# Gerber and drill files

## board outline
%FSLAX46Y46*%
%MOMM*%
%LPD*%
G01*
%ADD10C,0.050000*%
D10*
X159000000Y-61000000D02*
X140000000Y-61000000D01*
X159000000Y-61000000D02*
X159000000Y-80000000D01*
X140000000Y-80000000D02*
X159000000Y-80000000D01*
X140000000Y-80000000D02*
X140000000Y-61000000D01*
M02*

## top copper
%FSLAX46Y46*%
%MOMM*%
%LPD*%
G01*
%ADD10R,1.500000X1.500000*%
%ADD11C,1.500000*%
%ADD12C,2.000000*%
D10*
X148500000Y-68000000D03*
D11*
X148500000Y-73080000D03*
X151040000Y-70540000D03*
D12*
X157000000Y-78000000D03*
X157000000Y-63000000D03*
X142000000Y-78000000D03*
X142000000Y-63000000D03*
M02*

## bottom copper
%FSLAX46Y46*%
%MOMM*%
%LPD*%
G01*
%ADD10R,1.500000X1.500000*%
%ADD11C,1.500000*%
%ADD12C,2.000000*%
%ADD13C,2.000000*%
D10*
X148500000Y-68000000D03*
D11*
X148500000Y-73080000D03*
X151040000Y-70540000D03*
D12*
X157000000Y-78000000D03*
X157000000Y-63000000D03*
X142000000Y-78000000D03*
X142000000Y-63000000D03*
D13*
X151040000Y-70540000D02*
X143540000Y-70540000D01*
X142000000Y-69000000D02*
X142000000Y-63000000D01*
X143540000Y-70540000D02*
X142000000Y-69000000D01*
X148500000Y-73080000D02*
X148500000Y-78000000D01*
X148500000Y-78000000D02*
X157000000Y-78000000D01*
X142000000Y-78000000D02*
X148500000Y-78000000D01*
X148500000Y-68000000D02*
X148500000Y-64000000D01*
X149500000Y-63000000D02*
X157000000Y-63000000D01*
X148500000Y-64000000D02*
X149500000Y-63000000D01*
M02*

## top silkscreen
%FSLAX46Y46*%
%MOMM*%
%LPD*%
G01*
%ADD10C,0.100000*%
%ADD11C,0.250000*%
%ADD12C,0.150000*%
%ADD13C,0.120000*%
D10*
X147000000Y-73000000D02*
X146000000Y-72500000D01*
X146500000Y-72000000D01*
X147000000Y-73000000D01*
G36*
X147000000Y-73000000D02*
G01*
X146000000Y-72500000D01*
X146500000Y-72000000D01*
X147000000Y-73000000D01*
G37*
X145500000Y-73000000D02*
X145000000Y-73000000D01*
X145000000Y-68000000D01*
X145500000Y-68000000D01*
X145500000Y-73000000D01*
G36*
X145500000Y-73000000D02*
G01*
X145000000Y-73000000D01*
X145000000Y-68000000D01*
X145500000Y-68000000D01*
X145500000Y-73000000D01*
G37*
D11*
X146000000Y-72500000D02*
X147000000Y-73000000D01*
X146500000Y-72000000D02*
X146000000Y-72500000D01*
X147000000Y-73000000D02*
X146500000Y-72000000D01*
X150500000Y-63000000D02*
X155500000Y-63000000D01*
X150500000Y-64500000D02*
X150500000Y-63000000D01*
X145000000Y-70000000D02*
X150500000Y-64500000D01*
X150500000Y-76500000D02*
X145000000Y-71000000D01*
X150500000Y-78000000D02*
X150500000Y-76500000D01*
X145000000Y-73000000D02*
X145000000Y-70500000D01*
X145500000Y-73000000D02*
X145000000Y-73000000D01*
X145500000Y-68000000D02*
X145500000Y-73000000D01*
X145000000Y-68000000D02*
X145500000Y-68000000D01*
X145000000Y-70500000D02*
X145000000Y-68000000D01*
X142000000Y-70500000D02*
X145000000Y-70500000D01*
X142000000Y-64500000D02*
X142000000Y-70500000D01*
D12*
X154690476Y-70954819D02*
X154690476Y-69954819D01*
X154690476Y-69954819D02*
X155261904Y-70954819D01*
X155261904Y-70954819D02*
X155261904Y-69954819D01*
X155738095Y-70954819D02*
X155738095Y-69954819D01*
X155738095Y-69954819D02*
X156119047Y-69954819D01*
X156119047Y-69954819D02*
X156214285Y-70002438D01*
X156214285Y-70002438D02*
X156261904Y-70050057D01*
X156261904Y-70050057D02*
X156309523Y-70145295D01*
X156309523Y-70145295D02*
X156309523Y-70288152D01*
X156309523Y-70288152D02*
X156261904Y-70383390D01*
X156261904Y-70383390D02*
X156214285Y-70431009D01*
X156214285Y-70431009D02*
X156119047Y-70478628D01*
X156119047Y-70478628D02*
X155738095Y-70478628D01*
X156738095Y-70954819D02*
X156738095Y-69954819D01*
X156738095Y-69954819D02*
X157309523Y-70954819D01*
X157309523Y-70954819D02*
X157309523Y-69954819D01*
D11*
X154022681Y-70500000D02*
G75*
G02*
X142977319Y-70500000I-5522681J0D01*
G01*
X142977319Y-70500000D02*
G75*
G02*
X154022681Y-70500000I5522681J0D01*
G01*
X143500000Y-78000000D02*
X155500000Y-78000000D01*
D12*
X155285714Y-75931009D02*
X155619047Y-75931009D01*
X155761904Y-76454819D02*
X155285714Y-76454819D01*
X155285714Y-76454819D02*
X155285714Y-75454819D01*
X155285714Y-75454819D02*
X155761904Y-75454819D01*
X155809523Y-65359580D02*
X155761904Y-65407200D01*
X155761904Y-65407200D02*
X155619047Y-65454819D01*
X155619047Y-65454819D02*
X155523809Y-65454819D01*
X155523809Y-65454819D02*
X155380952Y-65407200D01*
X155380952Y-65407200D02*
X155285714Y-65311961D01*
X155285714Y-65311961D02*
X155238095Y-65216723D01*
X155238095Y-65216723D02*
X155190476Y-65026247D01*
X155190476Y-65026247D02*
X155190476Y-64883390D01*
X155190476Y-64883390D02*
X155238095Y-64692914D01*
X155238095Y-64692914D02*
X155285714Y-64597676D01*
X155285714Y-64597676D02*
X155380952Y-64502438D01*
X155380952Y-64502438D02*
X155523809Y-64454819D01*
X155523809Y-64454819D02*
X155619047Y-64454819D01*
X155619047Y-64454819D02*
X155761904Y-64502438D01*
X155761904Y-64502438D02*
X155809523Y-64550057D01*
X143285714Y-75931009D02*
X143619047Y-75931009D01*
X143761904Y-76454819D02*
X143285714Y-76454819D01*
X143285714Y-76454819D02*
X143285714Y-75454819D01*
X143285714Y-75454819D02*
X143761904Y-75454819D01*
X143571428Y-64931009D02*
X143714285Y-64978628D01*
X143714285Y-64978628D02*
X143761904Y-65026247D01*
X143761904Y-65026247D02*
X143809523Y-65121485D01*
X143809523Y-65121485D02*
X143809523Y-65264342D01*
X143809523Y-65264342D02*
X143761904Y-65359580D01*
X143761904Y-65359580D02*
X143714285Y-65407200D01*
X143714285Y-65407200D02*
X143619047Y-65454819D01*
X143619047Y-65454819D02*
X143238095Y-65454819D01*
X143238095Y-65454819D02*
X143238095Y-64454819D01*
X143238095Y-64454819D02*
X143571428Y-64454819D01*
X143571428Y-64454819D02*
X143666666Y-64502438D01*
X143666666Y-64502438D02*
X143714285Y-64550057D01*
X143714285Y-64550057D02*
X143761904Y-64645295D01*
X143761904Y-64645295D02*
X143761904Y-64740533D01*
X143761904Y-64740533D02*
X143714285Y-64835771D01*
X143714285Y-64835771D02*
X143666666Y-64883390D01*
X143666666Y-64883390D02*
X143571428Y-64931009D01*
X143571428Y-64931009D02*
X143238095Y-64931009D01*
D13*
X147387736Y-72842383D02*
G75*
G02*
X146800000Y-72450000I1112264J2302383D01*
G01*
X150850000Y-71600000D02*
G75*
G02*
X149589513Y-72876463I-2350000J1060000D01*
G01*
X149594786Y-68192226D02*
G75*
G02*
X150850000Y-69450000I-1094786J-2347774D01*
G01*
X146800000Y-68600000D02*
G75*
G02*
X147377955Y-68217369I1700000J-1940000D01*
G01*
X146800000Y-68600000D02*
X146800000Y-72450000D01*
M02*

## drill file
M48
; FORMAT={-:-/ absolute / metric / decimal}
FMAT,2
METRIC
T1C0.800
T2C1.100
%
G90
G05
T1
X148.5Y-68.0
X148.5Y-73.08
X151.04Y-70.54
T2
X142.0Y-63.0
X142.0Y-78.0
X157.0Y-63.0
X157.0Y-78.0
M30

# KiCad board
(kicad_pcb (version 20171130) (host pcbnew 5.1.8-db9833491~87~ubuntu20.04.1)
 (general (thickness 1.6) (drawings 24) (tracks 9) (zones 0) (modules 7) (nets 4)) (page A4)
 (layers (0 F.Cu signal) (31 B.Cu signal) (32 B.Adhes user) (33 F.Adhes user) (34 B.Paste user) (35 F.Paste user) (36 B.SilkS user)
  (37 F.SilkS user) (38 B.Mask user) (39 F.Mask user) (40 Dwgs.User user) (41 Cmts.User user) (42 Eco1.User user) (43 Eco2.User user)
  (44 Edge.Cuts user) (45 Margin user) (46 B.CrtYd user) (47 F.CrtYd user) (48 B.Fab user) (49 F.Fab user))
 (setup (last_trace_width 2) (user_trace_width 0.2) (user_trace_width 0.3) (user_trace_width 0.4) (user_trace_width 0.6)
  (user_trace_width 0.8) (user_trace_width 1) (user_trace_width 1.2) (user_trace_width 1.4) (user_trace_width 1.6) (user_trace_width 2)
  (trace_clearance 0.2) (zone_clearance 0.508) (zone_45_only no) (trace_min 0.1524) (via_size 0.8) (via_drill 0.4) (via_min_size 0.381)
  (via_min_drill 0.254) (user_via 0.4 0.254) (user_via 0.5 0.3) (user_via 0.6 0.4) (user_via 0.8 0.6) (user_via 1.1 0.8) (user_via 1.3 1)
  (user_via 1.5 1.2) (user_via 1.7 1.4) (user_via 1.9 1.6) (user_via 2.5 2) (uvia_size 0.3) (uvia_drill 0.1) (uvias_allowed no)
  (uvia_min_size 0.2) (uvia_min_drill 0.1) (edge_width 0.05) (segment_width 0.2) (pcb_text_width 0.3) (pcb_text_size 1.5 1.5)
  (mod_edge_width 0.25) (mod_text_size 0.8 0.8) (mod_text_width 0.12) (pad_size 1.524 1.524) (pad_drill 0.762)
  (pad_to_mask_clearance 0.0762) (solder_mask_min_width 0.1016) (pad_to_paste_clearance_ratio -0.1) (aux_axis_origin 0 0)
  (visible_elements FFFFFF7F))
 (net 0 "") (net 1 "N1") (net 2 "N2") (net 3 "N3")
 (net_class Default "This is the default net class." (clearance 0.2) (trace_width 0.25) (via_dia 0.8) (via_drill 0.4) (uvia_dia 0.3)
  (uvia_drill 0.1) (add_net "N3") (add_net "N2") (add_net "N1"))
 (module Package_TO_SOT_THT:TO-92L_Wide (layer F.Cu) (at 148.5 68 270)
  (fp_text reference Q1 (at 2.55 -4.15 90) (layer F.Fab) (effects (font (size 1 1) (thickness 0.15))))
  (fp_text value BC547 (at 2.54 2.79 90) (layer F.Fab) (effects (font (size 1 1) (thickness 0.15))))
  (fp_arc (start 2.54 0) (end 4.45 1.7) (angle -15.88591585) (layer F.SilkS) (width 0.12))
  (fp_arc (start 2.54 0) (end 3.6 -2.35) (angle 40.72153779) (layer F.SilkS) (width 0.12))
  (fp_arc (start 2.54 0) (end 1.45 -2.35) (angle -40.11670855) (layer F.SilkS) (width 0.12))
  (fp_arc (start 2.54 0) (end 0.6 1.7) (angle 15.44288892) (layer F.SilkS) (width 0.12))
  (fp_line (start 0.6 1.7) (end 4.45 1.7) (layer F.SilkS) (width 0.12))
  (pad 1 thru_hole rect (at 0 0 270) (size 1.5 1.5) (drill 0.8) (layers *.Cu *.Mask) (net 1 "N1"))
  (pad 3 thru_hole circle (at 5.08 0 270) (size 1.5 1.5) (drill 0.8) (layers *.Cu *.Mask) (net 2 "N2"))
  (pad 2 thru_hole circle (at 2.54 -2.54 270) (size 1.5 1.5) (drill 0.8) (layers *.Cu *.Mask) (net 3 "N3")))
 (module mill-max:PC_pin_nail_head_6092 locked (layer F.Cu) (at 157 78)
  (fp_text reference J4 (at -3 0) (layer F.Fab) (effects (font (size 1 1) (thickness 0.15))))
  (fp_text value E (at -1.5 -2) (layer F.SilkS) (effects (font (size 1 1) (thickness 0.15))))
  (pad 1 thru_hole circle (at 0 0) (size 2 2) (drill 1.1) (layers *.Cu *.Mask) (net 2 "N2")))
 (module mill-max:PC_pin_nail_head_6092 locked (layer F.Cu) (at 157 63)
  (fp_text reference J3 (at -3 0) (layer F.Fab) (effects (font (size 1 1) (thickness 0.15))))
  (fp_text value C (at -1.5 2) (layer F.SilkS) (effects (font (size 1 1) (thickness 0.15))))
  (pad 1 thru_hole circle (at 0 0) (size 2 2) (drill 1.1) (layers *.Cu *.Mask) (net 1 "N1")))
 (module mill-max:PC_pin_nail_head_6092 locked (layer F.Cu) (at 142 78)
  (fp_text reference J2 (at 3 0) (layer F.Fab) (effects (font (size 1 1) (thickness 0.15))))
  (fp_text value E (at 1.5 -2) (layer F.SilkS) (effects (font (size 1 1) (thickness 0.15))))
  (pad 1 thru_hole circle (at 0 0) (size 2 2) (drill 1.1) (layers *.Cu *.Mask) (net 2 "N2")))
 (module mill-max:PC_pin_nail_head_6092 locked (layer F.Cu) (at 142 63)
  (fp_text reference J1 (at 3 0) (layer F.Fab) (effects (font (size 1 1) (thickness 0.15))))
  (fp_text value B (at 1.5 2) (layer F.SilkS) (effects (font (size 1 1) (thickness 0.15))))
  (pad 1 thru_hole circle (at 0 0) (size 2 2) (drill 1.1) (layers *.Cu *.Mask) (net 3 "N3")))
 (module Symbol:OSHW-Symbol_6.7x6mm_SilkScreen (layer B.Cu) (at 155.5 70.5 270)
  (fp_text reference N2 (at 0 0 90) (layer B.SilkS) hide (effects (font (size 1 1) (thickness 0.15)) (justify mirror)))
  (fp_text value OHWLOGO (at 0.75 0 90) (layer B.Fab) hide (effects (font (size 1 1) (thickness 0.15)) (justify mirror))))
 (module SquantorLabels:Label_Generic (layer B.Cu) (at 141.5 71.5 90)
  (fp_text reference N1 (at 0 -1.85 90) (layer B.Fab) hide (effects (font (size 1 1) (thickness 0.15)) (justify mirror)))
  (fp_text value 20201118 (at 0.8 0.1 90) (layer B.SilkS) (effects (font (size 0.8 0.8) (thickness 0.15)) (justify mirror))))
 (gr_poly (pts (xy 147 73) (xy 146 72.5) (xy 146.5 72)) (layer F.SilkS) (width 0.1))
 (gr_poly (pts (xy 145.5 73) (xy 145 73) (xy 145 68) (xy 145.5 68)) (layer F.SilkS) (width 0.1))
 (gr_line (start 146 72.5) (end 147 73) (layer F.SilkS) (width 0.25))
 (gr_line (start 146.5 72) (end 146 72.5) (layer F.SilkS) (width 0.25))
 (gr_line (start 147 73) (end 146.5 72) (layer F.SilkS) (width 0.25))
 (gr_line (start 150.5 63) (end 155.5 63) (layer F.SilkS) (width 0.25))
 (gr_line (start 150.5 64.5) (end 150.5 63) (layer F.SilkS) (width 0.25))
 (gr_line (start 145 70) (end 150.5 64.5) (layer F.SilkS) (width 0.25))
 (gr_line (start 150.5 76.5) (end 145 71) (layer F.SilkS) (width 0.25))
 (gr_line (start 150.5 78) (end 150.5 76.5) (layer F.SilkS) (width 0.25))
 (gr_line (start 145 73) (end 145 70.5) (layer F.SilkS) (width 0.25))
 (gr_line (start 145.5 73) (end 145 73) (layer F.SilkS) (width 0.25))
 (gr_line (start 145.5 68) (end 145.5 73) (layer F.SilkS) (width 0.25))
 (gr_line (start 145 68) (end 145.5 68) (layer F.SilkS) (width 0.25))
 (gr_line (start 145 70.5) (end 145 68) (layer F.SilkS) (width 0.25))
 (gr_line (start 142 70.5) (end 145 70.5) (layer F.SilkS) (width 0.25))
 (gr_line (start 142 64.5) (end 142 70.5) (layer F.SilkS) (width 0.25))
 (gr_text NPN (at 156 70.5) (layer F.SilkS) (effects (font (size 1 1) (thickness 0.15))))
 (gr_circle (center 148.5 70.5) (end 154 71) (layer F.SilkS) (width 0.25))
 (gr_line (start 143.5 78) (end 155.5 78) (layer F.SilkS) (width 0.25))
 (gr_line (start 159 61) (end 140 61) (layer Edge.Cuts) (width 0.05))
 (gr_line (start 159 61) (end 159 80) (layer Edge.Cuts) (width 0.05))
 (gr_line (start 140 80) (end 159 80) (layer Edge.Cuts) (width 0.05))
 (gr_line (start 140 80) (end 140 61) (layer Edge.Cuts) (width 0.05))
 (segment (start 151.04 70.54) (end 143.54 70.54) (width 2) (layer B.Cu) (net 3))
 (segment (start 142 69) (end 142 63) (width 2) (layer B.Cu) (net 3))
 (segment (start 143.54 70.54) (end 142 69) (width 2) (layer B.Cu) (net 3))
 (segment (start 148.5 73.08) (end 148.5 78) (width 2) (layer B.Cu) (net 2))
 (segment (start 148.5 78) (end 157 78) (width 2) (layer B.Cu) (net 2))
 (segment (start 142 78) (end 148.5 78) (width 2) (layer B.Cu) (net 2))
 (segment (start 148.5 68) (end 148.5 64) (width 2) (layer B.Cu) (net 1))
 (segment (start 149.5 63) (end 157 63) (width 2) (layer B.Cu) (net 1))
 (segment (start 148.5 64) (end 149.5 63) (width 2) (layer B.Cu) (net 1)))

